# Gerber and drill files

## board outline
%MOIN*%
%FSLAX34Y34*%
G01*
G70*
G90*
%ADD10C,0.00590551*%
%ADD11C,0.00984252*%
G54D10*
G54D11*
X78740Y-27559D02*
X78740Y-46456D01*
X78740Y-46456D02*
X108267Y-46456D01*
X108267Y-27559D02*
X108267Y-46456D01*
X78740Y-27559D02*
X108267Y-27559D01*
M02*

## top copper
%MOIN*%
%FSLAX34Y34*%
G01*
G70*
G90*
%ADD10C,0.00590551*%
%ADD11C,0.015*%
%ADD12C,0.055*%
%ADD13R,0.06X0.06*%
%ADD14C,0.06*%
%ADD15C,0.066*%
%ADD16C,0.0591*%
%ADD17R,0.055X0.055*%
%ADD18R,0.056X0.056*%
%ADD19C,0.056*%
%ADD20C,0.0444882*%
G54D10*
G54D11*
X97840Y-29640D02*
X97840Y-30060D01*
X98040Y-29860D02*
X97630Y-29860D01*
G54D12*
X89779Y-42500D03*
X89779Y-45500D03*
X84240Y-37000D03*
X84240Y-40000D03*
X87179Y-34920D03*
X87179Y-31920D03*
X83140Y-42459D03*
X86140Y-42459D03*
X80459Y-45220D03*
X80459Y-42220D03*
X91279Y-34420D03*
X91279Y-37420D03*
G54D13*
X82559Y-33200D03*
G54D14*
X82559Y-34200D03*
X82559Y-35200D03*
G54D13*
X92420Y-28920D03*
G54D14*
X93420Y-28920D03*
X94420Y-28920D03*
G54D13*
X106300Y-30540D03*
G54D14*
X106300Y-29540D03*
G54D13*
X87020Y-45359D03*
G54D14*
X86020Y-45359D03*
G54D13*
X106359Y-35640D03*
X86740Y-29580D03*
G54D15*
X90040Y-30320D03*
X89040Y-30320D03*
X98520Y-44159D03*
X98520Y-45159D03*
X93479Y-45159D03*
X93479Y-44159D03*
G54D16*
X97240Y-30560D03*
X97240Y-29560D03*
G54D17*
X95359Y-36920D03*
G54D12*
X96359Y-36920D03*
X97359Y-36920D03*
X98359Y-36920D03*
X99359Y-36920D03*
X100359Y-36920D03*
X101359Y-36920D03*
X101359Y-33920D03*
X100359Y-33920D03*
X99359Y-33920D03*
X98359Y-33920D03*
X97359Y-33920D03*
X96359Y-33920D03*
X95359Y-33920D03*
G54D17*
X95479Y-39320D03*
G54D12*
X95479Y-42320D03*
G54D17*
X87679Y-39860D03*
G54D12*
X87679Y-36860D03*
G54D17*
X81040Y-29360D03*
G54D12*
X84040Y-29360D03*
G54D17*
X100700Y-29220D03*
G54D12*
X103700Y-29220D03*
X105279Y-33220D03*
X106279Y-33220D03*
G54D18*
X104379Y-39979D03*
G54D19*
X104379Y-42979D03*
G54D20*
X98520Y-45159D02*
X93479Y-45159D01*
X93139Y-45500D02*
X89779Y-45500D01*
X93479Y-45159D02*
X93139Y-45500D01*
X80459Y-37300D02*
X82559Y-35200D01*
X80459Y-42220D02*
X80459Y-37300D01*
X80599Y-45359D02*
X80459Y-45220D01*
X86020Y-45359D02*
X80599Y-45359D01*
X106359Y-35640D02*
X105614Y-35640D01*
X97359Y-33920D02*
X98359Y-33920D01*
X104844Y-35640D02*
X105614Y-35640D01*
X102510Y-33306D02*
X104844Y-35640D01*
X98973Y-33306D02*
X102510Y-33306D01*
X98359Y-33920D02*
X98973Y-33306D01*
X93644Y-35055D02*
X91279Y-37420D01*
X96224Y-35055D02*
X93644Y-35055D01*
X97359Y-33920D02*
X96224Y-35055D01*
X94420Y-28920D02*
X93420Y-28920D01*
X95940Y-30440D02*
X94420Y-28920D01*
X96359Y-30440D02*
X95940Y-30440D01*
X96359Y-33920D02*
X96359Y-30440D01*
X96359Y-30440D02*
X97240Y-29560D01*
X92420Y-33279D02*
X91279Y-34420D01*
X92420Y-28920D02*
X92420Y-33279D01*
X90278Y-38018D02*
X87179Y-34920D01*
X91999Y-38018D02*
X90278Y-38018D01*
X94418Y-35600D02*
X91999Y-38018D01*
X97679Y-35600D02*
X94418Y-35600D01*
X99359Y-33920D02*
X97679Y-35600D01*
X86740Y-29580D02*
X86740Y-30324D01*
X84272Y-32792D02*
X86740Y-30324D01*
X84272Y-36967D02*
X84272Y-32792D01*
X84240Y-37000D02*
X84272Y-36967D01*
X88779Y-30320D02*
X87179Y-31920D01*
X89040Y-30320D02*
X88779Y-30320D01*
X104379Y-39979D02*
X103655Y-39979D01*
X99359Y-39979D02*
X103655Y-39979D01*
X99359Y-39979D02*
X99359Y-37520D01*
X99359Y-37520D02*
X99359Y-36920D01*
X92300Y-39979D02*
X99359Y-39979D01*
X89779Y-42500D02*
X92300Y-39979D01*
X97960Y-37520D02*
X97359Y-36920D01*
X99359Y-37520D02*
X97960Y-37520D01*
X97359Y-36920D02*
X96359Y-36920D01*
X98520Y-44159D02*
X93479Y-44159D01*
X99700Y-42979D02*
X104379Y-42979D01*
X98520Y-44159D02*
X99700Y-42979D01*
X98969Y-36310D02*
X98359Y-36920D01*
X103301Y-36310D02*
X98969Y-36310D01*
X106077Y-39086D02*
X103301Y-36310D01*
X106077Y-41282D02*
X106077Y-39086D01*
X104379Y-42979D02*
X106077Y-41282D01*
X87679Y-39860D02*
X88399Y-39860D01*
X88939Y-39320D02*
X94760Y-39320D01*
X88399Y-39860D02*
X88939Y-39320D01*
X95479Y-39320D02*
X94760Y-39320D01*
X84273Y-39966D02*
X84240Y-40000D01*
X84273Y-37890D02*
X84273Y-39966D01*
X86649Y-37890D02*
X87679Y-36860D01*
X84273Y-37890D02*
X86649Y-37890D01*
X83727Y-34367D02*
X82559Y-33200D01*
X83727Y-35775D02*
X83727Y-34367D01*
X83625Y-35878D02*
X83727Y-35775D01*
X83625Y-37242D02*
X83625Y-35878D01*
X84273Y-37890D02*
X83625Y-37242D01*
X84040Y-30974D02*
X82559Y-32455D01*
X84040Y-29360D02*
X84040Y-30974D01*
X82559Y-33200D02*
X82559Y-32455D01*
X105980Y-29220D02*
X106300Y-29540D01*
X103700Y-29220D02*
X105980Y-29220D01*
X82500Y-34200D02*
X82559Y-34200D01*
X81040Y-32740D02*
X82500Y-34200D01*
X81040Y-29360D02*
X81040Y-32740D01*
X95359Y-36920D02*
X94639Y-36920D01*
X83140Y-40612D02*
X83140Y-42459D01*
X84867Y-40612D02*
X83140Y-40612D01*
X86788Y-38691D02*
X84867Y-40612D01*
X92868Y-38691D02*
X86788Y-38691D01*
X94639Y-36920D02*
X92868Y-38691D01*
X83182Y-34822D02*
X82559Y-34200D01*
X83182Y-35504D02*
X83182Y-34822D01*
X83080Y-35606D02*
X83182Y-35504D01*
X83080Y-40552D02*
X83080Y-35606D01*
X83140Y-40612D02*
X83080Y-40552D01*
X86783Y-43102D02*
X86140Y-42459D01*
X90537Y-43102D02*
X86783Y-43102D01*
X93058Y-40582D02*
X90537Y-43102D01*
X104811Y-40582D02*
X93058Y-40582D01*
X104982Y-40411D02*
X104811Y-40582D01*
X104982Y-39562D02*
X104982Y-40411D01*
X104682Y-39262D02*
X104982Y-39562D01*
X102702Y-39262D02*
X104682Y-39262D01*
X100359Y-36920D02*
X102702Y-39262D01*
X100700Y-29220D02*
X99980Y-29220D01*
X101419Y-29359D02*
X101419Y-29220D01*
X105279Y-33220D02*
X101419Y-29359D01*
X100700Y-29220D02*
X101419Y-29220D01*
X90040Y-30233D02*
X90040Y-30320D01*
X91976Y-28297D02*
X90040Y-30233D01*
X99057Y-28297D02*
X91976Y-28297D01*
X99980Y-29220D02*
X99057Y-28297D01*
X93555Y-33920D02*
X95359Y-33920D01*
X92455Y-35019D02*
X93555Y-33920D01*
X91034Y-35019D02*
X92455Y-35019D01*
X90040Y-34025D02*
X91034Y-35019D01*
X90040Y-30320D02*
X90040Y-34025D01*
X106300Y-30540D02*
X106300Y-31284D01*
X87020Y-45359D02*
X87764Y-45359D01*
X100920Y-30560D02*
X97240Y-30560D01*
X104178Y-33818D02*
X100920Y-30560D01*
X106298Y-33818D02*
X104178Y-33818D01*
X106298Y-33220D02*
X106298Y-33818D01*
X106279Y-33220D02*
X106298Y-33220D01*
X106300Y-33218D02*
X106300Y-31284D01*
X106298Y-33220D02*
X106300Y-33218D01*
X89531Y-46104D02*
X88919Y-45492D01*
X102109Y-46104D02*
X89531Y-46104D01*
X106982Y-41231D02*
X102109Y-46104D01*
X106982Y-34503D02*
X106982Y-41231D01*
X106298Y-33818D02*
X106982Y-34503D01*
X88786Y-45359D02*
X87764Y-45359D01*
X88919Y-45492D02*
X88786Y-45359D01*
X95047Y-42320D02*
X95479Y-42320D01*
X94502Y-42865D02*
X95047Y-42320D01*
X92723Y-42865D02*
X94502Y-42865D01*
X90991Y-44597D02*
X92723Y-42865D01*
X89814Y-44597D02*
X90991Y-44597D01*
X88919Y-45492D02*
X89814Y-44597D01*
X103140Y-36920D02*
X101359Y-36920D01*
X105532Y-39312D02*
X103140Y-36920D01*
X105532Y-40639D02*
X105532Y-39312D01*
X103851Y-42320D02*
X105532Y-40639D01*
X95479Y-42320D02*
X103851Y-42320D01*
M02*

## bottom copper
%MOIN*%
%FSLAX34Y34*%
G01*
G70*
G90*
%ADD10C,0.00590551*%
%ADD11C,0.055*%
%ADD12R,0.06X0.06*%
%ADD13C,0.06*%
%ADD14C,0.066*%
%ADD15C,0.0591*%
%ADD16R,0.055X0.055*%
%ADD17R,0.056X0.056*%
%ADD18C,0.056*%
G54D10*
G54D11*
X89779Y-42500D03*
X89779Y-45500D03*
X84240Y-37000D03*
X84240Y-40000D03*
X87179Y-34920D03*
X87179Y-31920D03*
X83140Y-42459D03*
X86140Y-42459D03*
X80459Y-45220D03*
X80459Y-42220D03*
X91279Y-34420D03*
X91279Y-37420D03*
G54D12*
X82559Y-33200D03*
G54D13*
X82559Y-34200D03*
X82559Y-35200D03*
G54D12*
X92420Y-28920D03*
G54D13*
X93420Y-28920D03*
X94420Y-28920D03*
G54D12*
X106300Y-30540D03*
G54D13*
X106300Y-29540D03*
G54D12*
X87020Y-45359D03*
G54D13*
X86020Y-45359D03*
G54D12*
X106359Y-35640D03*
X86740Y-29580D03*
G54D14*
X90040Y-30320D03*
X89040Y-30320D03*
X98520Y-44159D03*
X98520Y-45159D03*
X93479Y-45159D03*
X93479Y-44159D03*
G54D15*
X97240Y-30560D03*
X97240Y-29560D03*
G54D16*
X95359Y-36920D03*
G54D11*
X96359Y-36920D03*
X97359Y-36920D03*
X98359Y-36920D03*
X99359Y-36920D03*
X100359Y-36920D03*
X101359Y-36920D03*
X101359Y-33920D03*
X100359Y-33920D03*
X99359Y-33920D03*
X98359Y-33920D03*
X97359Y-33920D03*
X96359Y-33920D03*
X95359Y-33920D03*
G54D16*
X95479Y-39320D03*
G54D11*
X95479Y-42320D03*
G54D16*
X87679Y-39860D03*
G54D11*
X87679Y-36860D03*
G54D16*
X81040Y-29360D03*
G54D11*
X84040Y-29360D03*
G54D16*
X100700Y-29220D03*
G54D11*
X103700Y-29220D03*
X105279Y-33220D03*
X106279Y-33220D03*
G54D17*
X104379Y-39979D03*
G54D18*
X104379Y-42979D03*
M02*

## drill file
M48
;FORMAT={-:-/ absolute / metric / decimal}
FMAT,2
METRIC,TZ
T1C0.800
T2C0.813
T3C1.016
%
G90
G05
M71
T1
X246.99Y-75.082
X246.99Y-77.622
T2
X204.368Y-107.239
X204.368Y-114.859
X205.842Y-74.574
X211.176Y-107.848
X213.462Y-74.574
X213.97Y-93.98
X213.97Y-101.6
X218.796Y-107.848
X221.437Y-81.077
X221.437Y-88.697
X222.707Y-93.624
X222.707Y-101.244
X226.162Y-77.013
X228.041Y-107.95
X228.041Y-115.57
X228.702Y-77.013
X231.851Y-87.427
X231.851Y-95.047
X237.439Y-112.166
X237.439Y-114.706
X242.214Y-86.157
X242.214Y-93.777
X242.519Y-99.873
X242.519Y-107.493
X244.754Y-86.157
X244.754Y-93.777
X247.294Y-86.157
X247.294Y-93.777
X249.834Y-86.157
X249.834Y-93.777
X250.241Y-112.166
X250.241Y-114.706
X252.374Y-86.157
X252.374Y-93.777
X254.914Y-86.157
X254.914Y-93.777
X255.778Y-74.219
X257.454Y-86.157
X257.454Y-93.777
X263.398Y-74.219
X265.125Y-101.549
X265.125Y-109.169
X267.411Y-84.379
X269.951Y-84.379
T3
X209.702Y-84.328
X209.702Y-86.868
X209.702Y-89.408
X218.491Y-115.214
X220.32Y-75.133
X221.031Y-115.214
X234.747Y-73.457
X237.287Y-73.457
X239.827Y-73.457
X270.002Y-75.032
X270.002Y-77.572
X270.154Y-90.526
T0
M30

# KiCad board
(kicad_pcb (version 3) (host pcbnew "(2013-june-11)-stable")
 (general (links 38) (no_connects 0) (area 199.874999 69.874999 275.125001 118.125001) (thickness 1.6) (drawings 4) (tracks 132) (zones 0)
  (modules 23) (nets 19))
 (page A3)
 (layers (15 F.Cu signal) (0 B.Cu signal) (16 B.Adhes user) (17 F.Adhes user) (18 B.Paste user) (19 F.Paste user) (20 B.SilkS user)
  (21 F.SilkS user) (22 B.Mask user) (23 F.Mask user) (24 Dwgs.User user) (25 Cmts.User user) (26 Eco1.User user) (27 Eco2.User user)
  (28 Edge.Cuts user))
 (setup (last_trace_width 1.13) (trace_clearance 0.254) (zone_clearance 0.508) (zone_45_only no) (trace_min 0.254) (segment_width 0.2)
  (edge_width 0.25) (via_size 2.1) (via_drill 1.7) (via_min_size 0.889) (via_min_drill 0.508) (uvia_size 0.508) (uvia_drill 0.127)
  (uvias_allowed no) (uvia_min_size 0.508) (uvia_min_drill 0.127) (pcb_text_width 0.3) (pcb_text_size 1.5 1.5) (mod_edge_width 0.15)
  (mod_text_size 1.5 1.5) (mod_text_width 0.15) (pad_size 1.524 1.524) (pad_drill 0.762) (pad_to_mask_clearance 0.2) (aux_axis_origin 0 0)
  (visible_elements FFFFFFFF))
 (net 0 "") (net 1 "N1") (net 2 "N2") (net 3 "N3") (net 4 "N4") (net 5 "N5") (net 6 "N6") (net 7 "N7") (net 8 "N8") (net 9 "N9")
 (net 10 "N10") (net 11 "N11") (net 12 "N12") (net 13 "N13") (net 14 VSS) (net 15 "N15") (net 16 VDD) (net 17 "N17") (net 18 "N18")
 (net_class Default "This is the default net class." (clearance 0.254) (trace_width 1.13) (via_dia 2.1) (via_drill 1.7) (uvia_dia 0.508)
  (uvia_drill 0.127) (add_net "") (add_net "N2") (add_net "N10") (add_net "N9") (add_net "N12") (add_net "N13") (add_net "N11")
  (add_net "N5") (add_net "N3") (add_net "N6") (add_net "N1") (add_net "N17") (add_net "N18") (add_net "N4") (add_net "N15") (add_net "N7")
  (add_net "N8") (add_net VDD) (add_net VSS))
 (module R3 (layer F.Cu) (at 228.041 111.76 270) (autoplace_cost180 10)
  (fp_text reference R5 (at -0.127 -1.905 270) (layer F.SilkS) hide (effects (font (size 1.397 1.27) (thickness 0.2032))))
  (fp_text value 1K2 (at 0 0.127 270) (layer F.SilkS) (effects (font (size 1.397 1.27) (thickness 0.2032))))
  (pad 1 thru_hole circle (at -3.81 0 270) (size 1.397 1.397) (drill 0.8128) (layers *.Cu *.Mask F.SilkS) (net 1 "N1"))
  (pad 2 thru_hole circle (at 3.81 0 270) (size 1.397 1.397) (drill 0.8128) (layers *.Cu *.Mask F.SilkS) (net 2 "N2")))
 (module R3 (layer F.Cu) (at 213.97 97.79 270) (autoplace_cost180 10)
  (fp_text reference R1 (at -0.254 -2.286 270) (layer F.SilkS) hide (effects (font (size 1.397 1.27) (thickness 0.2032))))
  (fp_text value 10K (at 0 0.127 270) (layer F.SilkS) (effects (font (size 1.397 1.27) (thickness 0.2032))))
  (pad 1 thru_hole circle (at -3.81 0 270) (size 1.397 1.397) (drill 0.8128) (layers *.Cu *.Mask F.SilkS) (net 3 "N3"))
  (pad 2 thru_hole circle (at 3.81 0 270) (size 1.397 1.397) (drill 0.8128) (layers *.Cu *.Mask F.SilkS) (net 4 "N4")))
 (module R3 (layer F.Cu) (at 221.437 84.8868 90) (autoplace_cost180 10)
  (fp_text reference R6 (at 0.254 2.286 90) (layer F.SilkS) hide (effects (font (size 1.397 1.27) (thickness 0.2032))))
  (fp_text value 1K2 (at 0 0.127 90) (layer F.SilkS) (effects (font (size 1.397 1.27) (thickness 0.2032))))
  (pad 1 thru_hole circle (at -3.81 0 90) (size 1.397 1.397) (drill 0.8128) (layers *.Cu *.Mask F.SilkS) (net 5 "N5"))
  (pad 2 thru_hole circle (at 3.81 0 90) (size 1.397 1.397) (drill 0.8128) (layers *.Cu *.Mask F.SilkS) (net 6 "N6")))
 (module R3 (layer F.Cu) (at 214.986 107.848) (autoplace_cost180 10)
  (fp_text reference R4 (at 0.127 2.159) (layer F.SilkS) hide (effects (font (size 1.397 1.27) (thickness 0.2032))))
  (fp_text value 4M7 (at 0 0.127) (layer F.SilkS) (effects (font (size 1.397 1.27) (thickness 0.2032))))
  (pad 1 thru_hole circle (at -3.81 0) (size 1.397 1.397) (drill 0.8128) (layers *.Cu *.Mask F.SilkS) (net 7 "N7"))
  (pad 2 thru_hole circle (at 3.81 0) (size 1.397 1.397) (drill 0.8128) (layers *.Cu *.Mask F.SilkS) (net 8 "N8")))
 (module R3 (layer F.Cu) (at 204.368 111.049 90) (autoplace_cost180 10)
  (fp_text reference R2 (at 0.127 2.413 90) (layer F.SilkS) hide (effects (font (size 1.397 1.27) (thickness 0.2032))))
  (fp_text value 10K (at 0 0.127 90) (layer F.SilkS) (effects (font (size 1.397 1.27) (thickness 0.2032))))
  (pad 1 thru_hole circle (at -3.81 0 90) (size 1.397 1.397) (drill 0.8128) (layers *.Cu *.Mask F.SilkS) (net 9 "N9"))
  (pad 2 thru_hole circle (at 3.81 0 90) (size 1.397 1.397) (drill 0.8128) (layers *.Cu *.Mask F.SilkS) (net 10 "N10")))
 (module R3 (layer F.Cu) (at 231.851 91.2368 270) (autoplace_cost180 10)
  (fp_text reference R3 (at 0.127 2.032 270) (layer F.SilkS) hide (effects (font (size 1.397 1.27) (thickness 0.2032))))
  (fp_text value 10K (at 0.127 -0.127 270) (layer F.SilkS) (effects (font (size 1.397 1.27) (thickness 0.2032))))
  (pad 1 thru_hole circle (at -3.81 0 270) (size 1.397 1.397) (drill 0.8128) (layers *.Cu *.Mask F.SilkS) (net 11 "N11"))
  (pad 2 thru_hole circle (at 3.81 0 270) (size 1.397 1.397) (drill 0.8128) (layers *.Cu *.Mask F.SilkS) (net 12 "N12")))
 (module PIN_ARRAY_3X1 (layer F.Cu) (at 209.702 86.868 270)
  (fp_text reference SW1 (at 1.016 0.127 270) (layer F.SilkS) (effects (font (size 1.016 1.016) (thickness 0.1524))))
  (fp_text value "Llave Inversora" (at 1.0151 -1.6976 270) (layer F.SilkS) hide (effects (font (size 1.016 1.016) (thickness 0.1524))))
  (pad 1 thru_hole rect (at -2.54 0 270) (size 1.524 1.524) (drill 1.016) (layers *.Cu *.Mask F.SilkS) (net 4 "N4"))
  (pad 2 thru_hole circle (at 0 0 270) (size 1.524 1.524) (drill 1.016) (layers *.Cu *.Mask F.SilkS) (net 7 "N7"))
  (pad 3 thru_hole circle (at 2.54 0 270) (size 1.524 1.524) (drill 1.016) (layers *.Cu *.Mask F.SilkS) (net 10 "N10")))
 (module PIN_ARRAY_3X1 (layer F.Cu) (at 237.287 73.4568)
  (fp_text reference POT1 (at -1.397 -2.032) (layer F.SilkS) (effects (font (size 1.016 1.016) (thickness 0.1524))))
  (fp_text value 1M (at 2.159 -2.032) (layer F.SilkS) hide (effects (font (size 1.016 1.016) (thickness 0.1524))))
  (pad 1 thru_hole rect (at -2.54 0) (size 1.524 1.524) (drill 1.016) (layers *.Cu *.Mask F.SilkS) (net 11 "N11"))
  (pad 2 thru_hole circle (at 0 0) (size 1.524 1.524) (drill 1.016) (layers *.Cu *.Mask F.SilkS) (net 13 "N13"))
  (pad 3 thru_hole circle (at 2.54 0) (size 1.524 1.524) (drill 1.016) (layers *.Cu *.Mask F.SilkS) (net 13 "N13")))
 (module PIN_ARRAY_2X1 (layer F.Cu) (at 270.002 76.3016 90)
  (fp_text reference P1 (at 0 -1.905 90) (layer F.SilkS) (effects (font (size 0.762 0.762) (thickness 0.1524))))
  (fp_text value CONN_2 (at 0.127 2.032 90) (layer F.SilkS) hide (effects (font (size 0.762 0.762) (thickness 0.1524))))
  (pad 1 thru_hole rect (at -1.27 0 90) (size 1.524 1.524) (drill 1.016) (layers *.Cu *.Mask F.SilkS) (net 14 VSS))
  (pad 2 thru_hole circle (at 1.27 0 90) (size 1.524 1.524) (drill 1.016) (layers *.Cu *.Mask F.SilkS) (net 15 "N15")))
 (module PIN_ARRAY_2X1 (layer F.Cu) (at 219.761 115.214 180)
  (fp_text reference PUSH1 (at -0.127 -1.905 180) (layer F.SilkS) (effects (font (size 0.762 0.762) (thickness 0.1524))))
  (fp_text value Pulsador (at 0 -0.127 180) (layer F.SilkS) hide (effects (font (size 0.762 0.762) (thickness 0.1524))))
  (pad 1 thru_hole rect (at -1.27 0 180) (size 1.524 1.524) (drill 1.016) (layers *.Cu *.Mask F.SilkS) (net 14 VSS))
  (pad 2 thru_hole circle (at 1.27 0 180) (size 1.524 1.524) (drill 1.016) (layers *.Cu *.Mask F.SilkS) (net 9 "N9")))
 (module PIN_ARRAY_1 (layer F.Cu) (at 270.154 90.5256)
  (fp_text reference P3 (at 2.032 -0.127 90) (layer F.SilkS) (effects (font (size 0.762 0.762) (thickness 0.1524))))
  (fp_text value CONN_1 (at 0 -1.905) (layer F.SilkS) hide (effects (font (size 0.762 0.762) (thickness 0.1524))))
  (pad 1 thru_hole rect (at 0 0) (size 1.524 1.524) (drill 1.016) (layers *.Cu *.Mask F.SilkS) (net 12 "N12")))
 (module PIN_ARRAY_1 (layer F.Cu) (at 220.32 75.1332)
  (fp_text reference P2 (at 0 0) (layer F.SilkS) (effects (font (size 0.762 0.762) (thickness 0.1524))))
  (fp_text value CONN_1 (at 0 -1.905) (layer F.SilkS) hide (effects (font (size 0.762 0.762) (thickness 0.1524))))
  (pad 1 thru_hole rect (at 0 0) (size 1.524 1.524) (drill 1.016) (layers *.Cu *.Mask F.SilkS) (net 3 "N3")))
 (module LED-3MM (layer F.Cu) (at 227.432 77.0128 180)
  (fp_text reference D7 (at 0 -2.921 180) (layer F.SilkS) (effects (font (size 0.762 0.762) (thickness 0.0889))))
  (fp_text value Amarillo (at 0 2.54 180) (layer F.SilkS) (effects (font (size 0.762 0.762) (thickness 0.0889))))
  (pad 1 thru_hole circle (at -1.27 0 180) (size 1.6764 1.6764) (drill 0.8128) (layers *.Cu *.Mask F.SilkS) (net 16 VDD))
  (pad 2 thru_hole circle (at 1.27 0 180) (size 1.6764 1.6764) (drill 0.8128) (layers *.Cu *.Mask F.SilkS) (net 6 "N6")))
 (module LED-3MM (layer F.Cu) (at 250.241 113.436 270)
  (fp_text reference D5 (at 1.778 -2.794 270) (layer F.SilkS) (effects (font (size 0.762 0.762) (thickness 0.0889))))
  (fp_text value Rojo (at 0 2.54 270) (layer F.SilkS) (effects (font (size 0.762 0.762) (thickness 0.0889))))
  (pad 1 thru_hole circle (at -1.27 0 270) (size 1.6764 1.6764) (drill 0.8128) (layers *.Cu *.Mask F.SilkS) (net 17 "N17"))
  (pad 2 thru_hole circle (at 1.27 0 270) (size 1.6764 1.6764) (drill 0.8128) (layers *.Cu *.Mask F.SilkS) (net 2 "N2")))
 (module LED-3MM (layer F.Cu) (at 237.439 113.436 90)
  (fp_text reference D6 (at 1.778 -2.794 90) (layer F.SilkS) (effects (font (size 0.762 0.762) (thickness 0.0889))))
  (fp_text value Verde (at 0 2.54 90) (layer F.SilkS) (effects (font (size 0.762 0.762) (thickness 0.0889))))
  (pad 1 thru_hole circle (at -1.27 0 90) (size 1.6764 1.6764) (drill 0.8128) (layers *.Cu *.Mask F.SilkS) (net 2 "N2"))
  (pad 2 thru_hole circle (at 1.27 0 90) (size 1.6764 1.6764) (drill 0.8128) (layers *.Cu *.Mask F.SilkS) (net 17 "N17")))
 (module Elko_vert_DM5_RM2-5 (layer F.Cu) (at 246.99 76.3524 270)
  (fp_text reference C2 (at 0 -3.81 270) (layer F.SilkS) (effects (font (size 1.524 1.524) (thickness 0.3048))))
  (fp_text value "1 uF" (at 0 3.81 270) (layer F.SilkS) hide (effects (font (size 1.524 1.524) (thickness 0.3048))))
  (fp_line (start -1.0668 -1.524) (end 0 -1.524) (layer F.Cu) (width 0.381))
  (fp_line (start -0.508 -2.032) (end -0.508 -0.9906) (layer F.Cu) (width 0.381))
  (pad 2 thru_hole circle (at 1.27 0 270) (size 1.50114 1.50114) (drill 0.8001) (layers *.Cu *.Mask F.SilkS) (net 14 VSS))
  (pad 1 thru_hole circle (at -1.27 0 270) (size 1.50114 1.50114) (drill 0.8001) (layers *.Cu *.Mask F.SilkS) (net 13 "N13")))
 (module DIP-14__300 (layer F.Cu) (at 249.834 89.9668)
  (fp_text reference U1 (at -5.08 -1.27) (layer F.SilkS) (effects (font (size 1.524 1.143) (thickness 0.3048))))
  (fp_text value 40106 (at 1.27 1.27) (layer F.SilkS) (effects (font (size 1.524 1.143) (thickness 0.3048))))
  (pad 1 thru_hole rect (at -7.62 3.81) (size 1.397 1.397) (drill 0.8128) (layers *.Cu *.Mask F.SilkS) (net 7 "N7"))
  (pad 2 thru_hole circle (at -5.08 3.81) (size 1.397 1.397) (drill 0.8128) (layers *.Cu *.Mask F.SilkS) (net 1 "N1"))
  (pad 3 thru_hole circle (at -2.54 3.81) (size 1.397 1.397) (drill 0.8128) (layers *.Cu *.Mask F.SilkS) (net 1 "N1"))
  (pad 4 thru_hole circle (at 0 3.81) (size 1.397 1.397) (drill 0.8128) (layers *.Cu *.Mask F.SilkS) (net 17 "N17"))
  (pad 5 thru_hole circle (at 2.54 3.81) (size 1.397 1.397) (drill 0.8128) (layers *.Cu *.Mask F.SilkS) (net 1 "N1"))
  (pad 6 thru_hole circle (at 5.08 3.81) (size 1.397 1.397) (drill 0.8128) (layers *.Cu *.Mask F.SilkS) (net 8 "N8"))
  (pad 7 thru_hole circle (at 7.62 3.81) (size 1.397 1.397) (drill 0.8128) (layers *.Cu *.Mask F.SilkS) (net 14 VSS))
  (pad 8 thru_hole circle (at 7.62 -3.81) (size 1.397 1.397) (drill 0.8128) (layers *.Cu *.Mask F.SilkS))
  (pad 9 thru_hole circle (at 5.08 -3.81) (size 1.397 1.397) (drill 0.8128) (layers *.Cu *.Mask F.SilkS))
  (pad 10 thru_hole circle (at 2.54 -3.81) (size 1.397 1.397) (drill 0.8128) (layers *.Cu *.Mask F.SilkS) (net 5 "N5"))
  (pad 11 thru_hole circle (at 0 -3.81) (size 1.397 1.397) (drill 0.8128) (layers *.Cu *.Mask F.SilkS) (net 12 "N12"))
  (pad 12 thru_hole circle (at -2.54 -3.81) (size 1.397 1.397) (drill 0.8128) (layers *.Cu *.Mask F.SilkS) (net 12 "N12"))
  (pad 13 thru_hole circle (at -5.08 -3.81) (size 1.397 1.397) (drill 0.8128) (layers *.Cu *.Mask F.SilkS) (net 13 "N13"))
  (pad 14 thru_hole circle (at -7.62 -3.81) (size 1.397 1.397) (drill 0.8128) (layers *.Cu *.Mask F.SilkS) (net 16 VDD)))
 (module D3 (layer F.Cu) (at 242.519 103.683 90)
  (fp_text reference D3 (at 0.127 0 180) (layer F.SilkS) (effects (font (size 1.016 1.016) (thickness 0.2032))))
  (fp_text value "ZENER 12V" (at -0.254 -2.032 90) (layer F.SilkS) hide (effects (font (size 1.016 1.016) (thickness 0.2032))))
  (pad 2 thru_hole rect (at 3.81 0 90) (size 1.397 1.397) (drill 0.8128) (layers *.Cu *.Mask F.SilkS) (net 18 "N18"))
  (pad 1 thru_hole circle (at -3.81 0 90) (size 1.397 1.397) (drill 0.8128) (layers *.Cu *.Mask F.SilkS) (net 14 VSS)))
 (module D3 (layer F.Cu) (at 222.707 97.4344 270)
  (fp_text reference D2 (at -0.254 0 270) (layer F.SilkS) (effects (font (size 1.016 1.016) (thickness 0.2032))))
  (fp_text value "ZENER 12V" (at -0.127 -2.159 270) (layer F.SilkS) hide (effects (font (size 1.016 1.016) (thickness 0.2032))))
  (pad 2 thru_hole rect (at 3.81 0 270) (size 1.397 1.397) (drill 0.8128) (layers *.Cu *.Mask F.SilkS) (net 18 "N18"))
  (pad 1 thru_hole circle (at -3.81 0 270) (size 1.397 1.397) (drill 0.8128) (layers *.Cu *.Mask F.SilkS) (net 4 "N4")))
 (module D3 (layer F.Cu) (at 209.652 74.5744 180)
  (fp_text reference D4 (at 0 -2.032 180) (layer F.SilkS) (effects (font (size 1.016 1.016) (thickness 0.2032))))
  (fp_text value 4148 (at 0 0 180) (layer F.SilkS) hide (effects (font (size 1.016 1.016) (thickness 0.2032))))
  (pad 2 thru_hole rect (at 3.81 0 180) (size 1.397 1.397) (drill 0.8128) (layers *.Cu *.Mask F.SilkS) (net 7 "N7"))
  (pad 1 thru_hole circle (at -3.81 0 180) (size 1.397 1.397) (drill 0.8128) (layers *.Cu *.Mask F.SilkS) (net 4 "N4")))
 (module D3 (layer F.Cu) (at 259.588 74.2188 180)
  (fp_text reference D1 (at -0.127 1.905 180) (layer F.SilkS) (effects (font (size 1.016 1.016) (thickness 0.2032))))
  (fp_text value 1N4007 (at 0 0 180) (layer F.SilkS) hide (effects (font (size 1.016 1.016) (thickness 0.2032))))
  (pad 2 thru_hole rect (at 3.81 0 180) (size 1.397 1.397) (drill 0.8128) (layers *.Cu *.Mask F.SilkS) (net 16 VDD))
  (pad 1 thru_hole circle (at -3.81 0 180) (size 1.397 1.397) (drill 0.8128) (layers *.Cu *.Mask F.SilkS) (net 15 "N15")))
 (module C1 (layer F.Cu) (at 268.681 84.3788)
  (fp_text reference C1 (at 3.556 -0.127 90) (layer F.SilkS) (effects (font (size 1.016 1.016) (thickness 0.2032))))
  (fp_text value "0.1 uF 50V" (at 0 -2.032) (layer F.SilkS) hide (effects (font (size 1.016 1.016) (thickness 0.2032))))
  (pad 1 thru_hole circle (at -1.27 0) (size 1.397 1.397) (drill 0.8128) (layers *.Cu *.Mask F.SilkS) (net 16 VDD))
  (pad 2 thru_hole circle (at 1.27 0) (size 1.397 1.397) (drill 0.8128) (layers *.Cu *.Mask F.SilkS) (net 14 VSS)))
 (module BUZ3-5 (layer F.Cu) (at 265.125 105.359 270)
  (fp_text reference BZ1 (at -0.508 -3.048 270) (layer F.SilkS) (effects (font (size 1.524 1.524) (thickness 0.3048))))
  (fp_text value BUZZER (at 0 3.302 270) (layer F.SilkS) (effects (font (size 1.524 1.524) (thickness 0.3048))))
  (pad 1 thru_hole rect (at -3.81 0 270) (size 1.4224 1.4224) (drill 0.8128) (layers *.Cu *.Mask F.SilkS) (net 1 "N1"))
  (pad 2 thru_hole circle (at 3.81 0 270) (size 1.4224 1.4224) (drill 0.8128) (layers *.Cu *.Mask F.SilkS) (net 17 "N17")))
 (gr_line (start 200 70) (end 200 118) (angle 90) (layer Edge.Cuts) (width 0.25))
 (gr_line (start 200 118) (end 275 118) (angle 90) (layer Edge.Cuts) (width 0.25))
 (gr_line (start 275 70) (end 275 118) (angle 90) (layer Edge.Cuts) (width 0.25))
 (gr_line (start 200 70) (end 275 70) (angle 90) (layer Edge.Cuts) (width 0.25))
 (segment (start 250.241 114.706) (end 237.439 114.706) (width 1.13) (layer F.Cu) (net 2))
 (segment (start 236.575 115.57) (end 228.041 115.57) (width 1.13) (layer F.Cu) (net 2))
 (segment (start 237.439 114.706) (end 236.575 115.57) (width 1.13) (layer F.Cu) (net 2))
 (segment (start 204.368 94.742) (end 209.702 89.408) (width 1.13) (layer F.Cu) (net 10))
 (segment (start 204.368 107.239) (end 204.368 94.742) (width 1.13) (layer F.Cu) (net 10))
 (segment (start 204.723 115.214) (end 204.368 114.859) (width 1.13) (layer F.Cu) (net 9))
 (segment (start 218.491 115.214) (end 204.723 115.214) (width 1.13) (layer F.Cu) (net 9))
 (segment (start 270.154 90.5256) (end 268.262 90.5256) (width 1.13) (layer F.Cu) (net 12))
 (segment (start 247.294 86.1568) (end 249.834 86.1568) (width 1.13) (layer F.Cu) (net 12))
 (segment (start 266.3044 90.5256) (end 268.262 90.5256) (width 1.13) (layer F.Cu) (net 12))
 (segment (start 260.3774 84.5986) (end 266.3044 90.5256) (width 1.13) (layer F.Cu) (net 12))
 (segment (start 251.3922 84.5986) (end 260.3774 84.5986) (width 1.13) (layer F.Cu) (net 12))
 (segment (start 249.834 86.1568) (end 251.3922 84.5986) (width 1.13) (layer F.Cu) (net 12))
 (segment (start 237.8581 89.0397) (end 231.851 95.0468) (width 1.13) (layer F.Cu) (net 12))
 (segment (start 244.4111 89.0397) (end 237.8581 89.0397) (width 1.13) (layer F.Cu) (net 12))
 (segment (start 247.294 86.1568) (end 244.4111 89.0397) (width 1.13) (layer F.Cu) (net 12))
 (segment (start 239.827 73.4568) (end 237.287 73.4568) (width 1.13) (layer F.Cu) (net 13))
 (segment (start 243.6886 77.3184) (end 239.827 73.4568) (width 1.13) (layer F.Cu) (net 13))
 (segment (start 244.754 77.3184) (end 243.6886 77.3184) (width 1.13) (layer F.Cu) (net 13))
 (segment (start 244.754 86.1568) (end 244.754 77.3184) (width 1.13) (layer F.Cu) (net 13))
 (segment (start 244.754 77.3184) (end 246.99 75.0824) (width 1.13) (layer F.Cu) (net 13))
 (segment (start 234.747 84.5308) (end 231.851 87.4268) (width 1.13) (layer F.Cu) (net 11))
 (segment (start 234.747 73.4568) (end 234.747 84.5308) (width 1.13) (layer F.Cu) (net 11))
 (segment (start 229.3081 96.5679) (end 221.437 88.6968) (width 1.13) (layer F.Cu) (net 5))
 (segment (start 233.679 96.5679) (end 229.3081 96.5679) (width 1.13) (layer F.Cu) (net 5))
 (segment (start 239.8228 90.4241) (end 233.679 96.5679) (width 1.13) (layer F.Cu) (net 5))
 (segment (start 248.1067 90.4241) (end 239.8228 90.4241) (width 1.13) (layer F.Cu) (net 5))
 (segment (start 252.374 86.1568) (end 248.1067 90.4241) (width 1.13) (layer F.Cu) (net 5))
 (segment (start 220.32 75.1332) (end 220.32 77.0252) (width 1.13) (layer F.Cu) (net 3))
 (segment (start 214.052 83.2932) (end 220.32 77.0252) (width 1.13) (layer F.Cu) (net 3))
 (segment (start 214.052 93.898) (end 214.052 83.2932) (width 1.13) (layer F.Cu) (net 3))
 (segment (start 213.97 93.98) (end 214.052 93.898) (width 1.13) (layer F.Cu) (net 3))
 (segment (start 225.501 77.0128) (end 221.437 81.0768) (width 1.13) (layer F.Cu) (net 6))
 (segment (start 226.162 77.0128) (end 225.501 77.0128) (width 1.13) (layer F.Cu) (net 6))
 (segment (start 265.125 101.549) (end 263.2838 101.549) (width 1.13) (layer F.Cu) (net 1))
 (segment (start 252.374 101.549) (end 263.2838 101.549) (width 1.13) (layer F.Cu) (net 1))
 (segment (start 252.374 101.549) (end 252.374 95.3022) (width 1.13) (layer F.Cu) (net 1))
 (segment (start 252.374 95.3022) (end 252.374 93.7768) (width 1.13) (layer F.Cu) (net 1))
 (segment (start 234.442 101.549) (end 252.374 101.549) (width 1.13) (layer F.Cu) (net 1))
 (segment (start 228.041 107.95) (end 234.442 101.549) (width 1.13) (layer F.Cu) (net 1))
 (segment (start 248.8194 95.3022) (end 247.294 93.7768) (width 1.13) (layer F.Cu) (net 1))
 (segment (start 252.374 95.3022) (end 248.8194 95.3022) (width 1.13) (layer F.Cu) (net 1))
 (segment (start 247.294 93.7768) (end 244.754 93.7768) (width 1.13) (layer F.Cu) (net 1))
 (segment (start 250.241 112.166) (end 237.439 112.166) (width 1.13) (layer F.Cu) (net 17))
 (segment (start 253.238 109.169) (end 265.125 109.169) (width 1.13) (layer F.Cu) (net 17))
 (segment (start 250.241 112.166) (end 253.238 109.169) (width 1.13) (layer F.Cu) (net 17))
 (segment (start 251.3816 92.2292) (end 249.834 93.7768) (width 1.13) (layer F.Cu) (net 17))
 (segment (start 262.3868 92.2292) (end 251.3816 92.2292) (width 1.13) (layer F.Cu) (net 17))
 (segment (start 269.4367 99.2791) (end 262.3868 92.2292) (width 1.13) (layer F.Cu) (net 17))
 (segment (start 269.4367 104.8573) (end 269.4367 99.2791) (width 1.13) (layer F.Cu) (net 17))
 (segment (start 265.125 109.169) (end 269.4367 104.8573) (width 1.13) (layer F.Cu) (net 17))
 (segment (start 222.707 101.2444) (end 224.5355 101.2444) (width 1.13) (layer F.Cu) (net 18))
 (segment (start 225.9069 99.873) (end 240.6905 99.873) (width 1.13) (layer F.Cu) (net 18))
 (segment (start 224.5355 101.2444) (end 225.9069 99.873) (width 1.13) (layer F.Cu) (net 18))
 (segment (start 242.519 99.873) (end 240.6905 99.873) (width 1.13) (layer F.Cu) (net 18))
 (segment (start 214.0558 101.5142) (end 213.97 101.6) (width 1.13) (layer F.Cu) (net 4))
 (segment (start 214.0558 96.2426) (end 214.0558 101.5142) (width 1.13) (layer F.Cu) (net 4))
 (segment (start 220.0888 96.2426) (end 222.707 93.6244) (width 1.13) (layer F.Cu) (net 4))
 (segment (start 214.0558 96.2426) (end 220.0888 96.2426) (width 1.13) (layer F.Cu) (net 4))
 (segment (start 212.6677 87.2937) (end 209.702 84.328) (width 1.13) (layer F.Cu) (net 4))
 (segment (start 212.6677 90.8706) (end 212.6677 87.2937) (width 1.13) (layer F.Cu) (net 4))
 (segment (start 212.4081 91.1302) (end 212.6677 90.8706) (width 1.13) (layer F.Cu) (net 4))
 (segment (start 212.4081 94.5949) (end 212.4081 91.1302) (width 1.13) (layer F.Cu) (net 4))
 (segment (start 214.0558 96.2426) (end 212.4081 94.5949) (width 1.13) (layer F.Cu) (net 4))
 (segment (start 213.462 78.676) (end 209.702 82.436) (width 1.13) (layer F.Cu) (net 4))
 (segment (start 213.462 74.5744) (end 213.462 78.676) (width 1.13) (layer F.Cu) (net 4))
 (segment (start 209.702 84.328) (end 209.702 82.436) (width 1.13) (layer F.Cu) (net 4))
 (segment (start 269.1892 74.2188) (end 270.002 75.0316) (width 1.13) (layer F.Cu) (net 15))
 (segment (start 263.398 74.2188) (end 269.1892 74.2188) (width 1.13) (layer F.Cu) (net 15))
 (segment (start 209.5502 86.868) (end 209.702 86.868) (width 1.13) (layer F.Cu) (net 7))
 (segment (start 205.842 83.1598) (end 209.5502 86.868) (width 1.13) (layer F.Cu) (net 7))
 (segment (start 205.842 74.5744) (end 205.842 83.1598) (width 1.13) (layer F.Cu) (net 7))
 (segment (start 242.214 93.7768) (end 240.3855 93.7768) (width 1.13) (layer F.Cu) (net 7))
 (segment (start 211.176 103.1566) (end 211.176 107.848) (width 1.13) (layer F.Cu) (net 7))
 (segment (start 215.5628 103.1566) (end 211.176 103.1566) (width 1.13) (layer F.Cu) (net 7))
 (segment (start 220.4421 98.2773) (end 215.5628 103.1566) (width 1.13) (layer F.Cu) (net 7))
 (segment (start 235.885 98.2773) (end 220.4421 98.2773) (width 1.13) (layer F.Cu) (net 7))
 (segment (start 240.3855 93.7768) (end 235.885 98.2773) (width 1.13) (layer F.Cu) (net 7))
 (segment (start 211.2833 88.4493) (end 209.702 86.868) (width 1.13) (layer F.Cu) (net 7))
 (segment (start 211.2833 90.1802) (end 211.2833 88.4493) (width 1.13) (layer F.Cu) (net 7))
 (segment (start 211.0237 90.4398) (end 211.2833 90.1802) (width 1.13) (layer F.Cu) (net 7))
 (segment (start 211.0237 103.0043) (end 211.0237 90.4398) (width 1.13) (layer F.Cu) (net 7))
 (segment (start 211.176 103.1566) (end 211.0237 103.0043) (width 1.13) (layer F.Cu) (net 7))
 (segment (start 220.4292 109.4812) (end 218.796 107.848) (width 1.13) (layer F.Cu) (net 8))
 (segment (start 229.9662 109.4812) (end 220.4292 109.4812) (width 1.13) (layer F.Cu) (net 8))
 (segment (start 236.3678 103.0796) (end 229.9662 109.4812) (width 1.13) (layer F.Cu) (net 8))
 (segment (start 266.2224 103.0796) (end 236.3678 103.0796) (width 1.13) (layer F.Cu) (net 8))
 (segment (start 266.6556 102.6464) (end 266.2224 103.0796) (width 1.13) (layer F.Cu) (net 8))
 (segment (start 266.6556 100.4876) (end 266.6556 102.6464) (width 1.13) (layer F.Cu) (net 8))
 (segment (start 265.8945 99.7265) (end 266.6556 100.4876) (width 1.13) (layer F.Cu) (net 8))
 (segment (start 260.8637 99.7265) (end 265.8945 99.7265) (width 1.13) (layer F.Cu) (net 8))
 (segment (start 254.914 93.7768) (end 260.8637 99.7265) (width 1.13) (layer F.Cu) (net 8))
 (segment (start 255.778 74.2188) (end 253.9495 74.2188) (width 1.13) (layer F.Cu) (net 16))
 (segment (start 257.6065 74.5743) (end 257.6065 74.2188) (width 1.13) (layer F.Cu) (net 16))
 (segment (start 267.411 84.3788) (end 257.6065 74.5743) (width 1.13) (layer F.Cu) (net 16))
 (segment (start 255.778 74.2188) (end 257.6065 74.2188) (width 1.13) (layer F.Cu) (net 16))
 (segment (start 228.702 76.7937) (end 228.702 77.0128) (width 1.13) (layer F.Cu) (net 16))
 (segment (start 233.6203 71.8754) (end 228.702 76.7937) (width 1.13) (layer F.Cu) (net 16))
 (segment (start 251.6061 71.8754) (end 233.6203 71.8754) (width 1.13) (layer F.Cu) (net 16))
 (segment (start 253.9495 74.2188) (end 251.6061 71.8754) (width 1.13) (layer F.Cu) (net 16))
 (segment (start 237.6299 86.1568) (end 242.214 86.1568) (width 1.13) (layer F.Cu) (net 16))
 (segment (start 234.8365 88.9502) (end 237.6299 86.1568) (width 1.13) (layer F.Cu) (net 16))
 (segment (start 231.2279 88.9502) (end 234.8365 88.9502) (width 1.13) (layer F.Cu) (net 16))
 (segment (start 228.702 86.4243) (end 231.2279 88.9502) (width 1.13) (layer F.Cu) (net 16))
 (segment (start 228.702 77.0128) (end 228.702 86.4243) (width 1.13) (layer F.Cu) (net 16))
 (segment (start 270.002 77.5716) (end 270.002 79.4636) (width 1.13) (layer F.Cu) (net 14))
 (segment (start 221.031 115.214) (end 222.923 115.214) (width 1.13) (layer F.Cu) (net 14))
 (segment (start 256.3376 77.6224) (end 246.99 77.6224) (width 1.13) (layer F.Cu) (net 14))
 (segment (start 264.614 85.8988) (end 256.3376 77.6224) (width 1.13) (layer F.Cu) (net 14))
 (segment (start 269.9974 85.8988) (end 264.614 85.8988) (width 1.13) (layer F.Cu) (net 14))
 (segment (start 269.9974 84.3788) (end 269.9974 85.8988) (width 1.13) (layer F.Cu) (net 14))
 (segment (start 269.951 84.3788) (end 269.9974 84.3788) (width 1.13) (layer F.Cu) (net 14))
 (segment (start 270.002 84.3742) (end 270.002 79.4636) (width 1.13) (layer F.Cu) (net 14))
 (segment (start 269.9974 84.3788) (end 270.002 84.3742) (width 1.13) (layer F.Cu) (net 14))
 (segment (start 227.4104 117.106) (end 225.8549 115.5504) (width 1.13) (layer F.Cu) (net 14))
 (segment (start 259.3577 117.106) (end 227.4104 117.106) (width 1.13) (layer F.Cu) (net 14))
 (segment (start 271.7368 104.7269) (end 259.3577 117.106) (width 1.13) (layer F.Cu) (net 14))
 (segment (start 271.7368 87.6382) (end 271.7368 104.7269) (width 1.13) (layer F.Cu) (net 14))
 (segment (start 269.9974 85.8988) (end 271.7368 87.6382) (width 1.13) (layer F.Cu) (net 14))
 (segment (start 225.5184 115.214) (end 222.923 115.214) (width 1.13) (layer F.Cu) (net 14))
 (segment (start 225.8549 115.5504) (end 225.5184 115.214) (width 1.13) (layer F.Cu) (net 14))
 (segment (start 241.4203 107.493) (end 242.519 107.493) (width 1.13) (layer F.Cu) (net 14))
 (segment (start 240.036 108.8773) (end 241.4203 107.493) (width 1.13) (layer F.Cu) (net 14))
 (segment (start 235.5173 108.8773) (end 240.036 108.8773) (width 1.13) (layer F.Cu) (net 14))
 (segment (start 231.1173 113.2773) (end 235.5173 108.8773) (width 1.13) (layer F.Cu) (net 14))
 (segment (start 228.128 113.2773) (end 231.1173 113.2773) (width 1.13) (layer F.Cu) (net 14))
 (segment (start 225.8549 115.5504) (end 228.128 113.2773) (width 1.13) (layer F.Cu) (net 14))
 (segment (start 261.9765 93.7768) (end 257.454 93.7768) (width 1.13) (layer F.Cu) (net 14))
 (segment (start 268.0523 99.8526) (end 261.9765 93.7768) (width 1.13) (layer F.Cu) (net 14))
 (segment (start 268.0523 103.2242) (end 268.0523 99.8526) (width 1.13) (layer F.Cu) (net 14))
 (segment (start 263.7835 107.493) (end 268.0523 103.2242) (width 1.13) (layer F.Cu) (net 14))
 (segment (start 242.519 107.493) (end 263.7835 107.493) (width 1.13) (layer F.Cu) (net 14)))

